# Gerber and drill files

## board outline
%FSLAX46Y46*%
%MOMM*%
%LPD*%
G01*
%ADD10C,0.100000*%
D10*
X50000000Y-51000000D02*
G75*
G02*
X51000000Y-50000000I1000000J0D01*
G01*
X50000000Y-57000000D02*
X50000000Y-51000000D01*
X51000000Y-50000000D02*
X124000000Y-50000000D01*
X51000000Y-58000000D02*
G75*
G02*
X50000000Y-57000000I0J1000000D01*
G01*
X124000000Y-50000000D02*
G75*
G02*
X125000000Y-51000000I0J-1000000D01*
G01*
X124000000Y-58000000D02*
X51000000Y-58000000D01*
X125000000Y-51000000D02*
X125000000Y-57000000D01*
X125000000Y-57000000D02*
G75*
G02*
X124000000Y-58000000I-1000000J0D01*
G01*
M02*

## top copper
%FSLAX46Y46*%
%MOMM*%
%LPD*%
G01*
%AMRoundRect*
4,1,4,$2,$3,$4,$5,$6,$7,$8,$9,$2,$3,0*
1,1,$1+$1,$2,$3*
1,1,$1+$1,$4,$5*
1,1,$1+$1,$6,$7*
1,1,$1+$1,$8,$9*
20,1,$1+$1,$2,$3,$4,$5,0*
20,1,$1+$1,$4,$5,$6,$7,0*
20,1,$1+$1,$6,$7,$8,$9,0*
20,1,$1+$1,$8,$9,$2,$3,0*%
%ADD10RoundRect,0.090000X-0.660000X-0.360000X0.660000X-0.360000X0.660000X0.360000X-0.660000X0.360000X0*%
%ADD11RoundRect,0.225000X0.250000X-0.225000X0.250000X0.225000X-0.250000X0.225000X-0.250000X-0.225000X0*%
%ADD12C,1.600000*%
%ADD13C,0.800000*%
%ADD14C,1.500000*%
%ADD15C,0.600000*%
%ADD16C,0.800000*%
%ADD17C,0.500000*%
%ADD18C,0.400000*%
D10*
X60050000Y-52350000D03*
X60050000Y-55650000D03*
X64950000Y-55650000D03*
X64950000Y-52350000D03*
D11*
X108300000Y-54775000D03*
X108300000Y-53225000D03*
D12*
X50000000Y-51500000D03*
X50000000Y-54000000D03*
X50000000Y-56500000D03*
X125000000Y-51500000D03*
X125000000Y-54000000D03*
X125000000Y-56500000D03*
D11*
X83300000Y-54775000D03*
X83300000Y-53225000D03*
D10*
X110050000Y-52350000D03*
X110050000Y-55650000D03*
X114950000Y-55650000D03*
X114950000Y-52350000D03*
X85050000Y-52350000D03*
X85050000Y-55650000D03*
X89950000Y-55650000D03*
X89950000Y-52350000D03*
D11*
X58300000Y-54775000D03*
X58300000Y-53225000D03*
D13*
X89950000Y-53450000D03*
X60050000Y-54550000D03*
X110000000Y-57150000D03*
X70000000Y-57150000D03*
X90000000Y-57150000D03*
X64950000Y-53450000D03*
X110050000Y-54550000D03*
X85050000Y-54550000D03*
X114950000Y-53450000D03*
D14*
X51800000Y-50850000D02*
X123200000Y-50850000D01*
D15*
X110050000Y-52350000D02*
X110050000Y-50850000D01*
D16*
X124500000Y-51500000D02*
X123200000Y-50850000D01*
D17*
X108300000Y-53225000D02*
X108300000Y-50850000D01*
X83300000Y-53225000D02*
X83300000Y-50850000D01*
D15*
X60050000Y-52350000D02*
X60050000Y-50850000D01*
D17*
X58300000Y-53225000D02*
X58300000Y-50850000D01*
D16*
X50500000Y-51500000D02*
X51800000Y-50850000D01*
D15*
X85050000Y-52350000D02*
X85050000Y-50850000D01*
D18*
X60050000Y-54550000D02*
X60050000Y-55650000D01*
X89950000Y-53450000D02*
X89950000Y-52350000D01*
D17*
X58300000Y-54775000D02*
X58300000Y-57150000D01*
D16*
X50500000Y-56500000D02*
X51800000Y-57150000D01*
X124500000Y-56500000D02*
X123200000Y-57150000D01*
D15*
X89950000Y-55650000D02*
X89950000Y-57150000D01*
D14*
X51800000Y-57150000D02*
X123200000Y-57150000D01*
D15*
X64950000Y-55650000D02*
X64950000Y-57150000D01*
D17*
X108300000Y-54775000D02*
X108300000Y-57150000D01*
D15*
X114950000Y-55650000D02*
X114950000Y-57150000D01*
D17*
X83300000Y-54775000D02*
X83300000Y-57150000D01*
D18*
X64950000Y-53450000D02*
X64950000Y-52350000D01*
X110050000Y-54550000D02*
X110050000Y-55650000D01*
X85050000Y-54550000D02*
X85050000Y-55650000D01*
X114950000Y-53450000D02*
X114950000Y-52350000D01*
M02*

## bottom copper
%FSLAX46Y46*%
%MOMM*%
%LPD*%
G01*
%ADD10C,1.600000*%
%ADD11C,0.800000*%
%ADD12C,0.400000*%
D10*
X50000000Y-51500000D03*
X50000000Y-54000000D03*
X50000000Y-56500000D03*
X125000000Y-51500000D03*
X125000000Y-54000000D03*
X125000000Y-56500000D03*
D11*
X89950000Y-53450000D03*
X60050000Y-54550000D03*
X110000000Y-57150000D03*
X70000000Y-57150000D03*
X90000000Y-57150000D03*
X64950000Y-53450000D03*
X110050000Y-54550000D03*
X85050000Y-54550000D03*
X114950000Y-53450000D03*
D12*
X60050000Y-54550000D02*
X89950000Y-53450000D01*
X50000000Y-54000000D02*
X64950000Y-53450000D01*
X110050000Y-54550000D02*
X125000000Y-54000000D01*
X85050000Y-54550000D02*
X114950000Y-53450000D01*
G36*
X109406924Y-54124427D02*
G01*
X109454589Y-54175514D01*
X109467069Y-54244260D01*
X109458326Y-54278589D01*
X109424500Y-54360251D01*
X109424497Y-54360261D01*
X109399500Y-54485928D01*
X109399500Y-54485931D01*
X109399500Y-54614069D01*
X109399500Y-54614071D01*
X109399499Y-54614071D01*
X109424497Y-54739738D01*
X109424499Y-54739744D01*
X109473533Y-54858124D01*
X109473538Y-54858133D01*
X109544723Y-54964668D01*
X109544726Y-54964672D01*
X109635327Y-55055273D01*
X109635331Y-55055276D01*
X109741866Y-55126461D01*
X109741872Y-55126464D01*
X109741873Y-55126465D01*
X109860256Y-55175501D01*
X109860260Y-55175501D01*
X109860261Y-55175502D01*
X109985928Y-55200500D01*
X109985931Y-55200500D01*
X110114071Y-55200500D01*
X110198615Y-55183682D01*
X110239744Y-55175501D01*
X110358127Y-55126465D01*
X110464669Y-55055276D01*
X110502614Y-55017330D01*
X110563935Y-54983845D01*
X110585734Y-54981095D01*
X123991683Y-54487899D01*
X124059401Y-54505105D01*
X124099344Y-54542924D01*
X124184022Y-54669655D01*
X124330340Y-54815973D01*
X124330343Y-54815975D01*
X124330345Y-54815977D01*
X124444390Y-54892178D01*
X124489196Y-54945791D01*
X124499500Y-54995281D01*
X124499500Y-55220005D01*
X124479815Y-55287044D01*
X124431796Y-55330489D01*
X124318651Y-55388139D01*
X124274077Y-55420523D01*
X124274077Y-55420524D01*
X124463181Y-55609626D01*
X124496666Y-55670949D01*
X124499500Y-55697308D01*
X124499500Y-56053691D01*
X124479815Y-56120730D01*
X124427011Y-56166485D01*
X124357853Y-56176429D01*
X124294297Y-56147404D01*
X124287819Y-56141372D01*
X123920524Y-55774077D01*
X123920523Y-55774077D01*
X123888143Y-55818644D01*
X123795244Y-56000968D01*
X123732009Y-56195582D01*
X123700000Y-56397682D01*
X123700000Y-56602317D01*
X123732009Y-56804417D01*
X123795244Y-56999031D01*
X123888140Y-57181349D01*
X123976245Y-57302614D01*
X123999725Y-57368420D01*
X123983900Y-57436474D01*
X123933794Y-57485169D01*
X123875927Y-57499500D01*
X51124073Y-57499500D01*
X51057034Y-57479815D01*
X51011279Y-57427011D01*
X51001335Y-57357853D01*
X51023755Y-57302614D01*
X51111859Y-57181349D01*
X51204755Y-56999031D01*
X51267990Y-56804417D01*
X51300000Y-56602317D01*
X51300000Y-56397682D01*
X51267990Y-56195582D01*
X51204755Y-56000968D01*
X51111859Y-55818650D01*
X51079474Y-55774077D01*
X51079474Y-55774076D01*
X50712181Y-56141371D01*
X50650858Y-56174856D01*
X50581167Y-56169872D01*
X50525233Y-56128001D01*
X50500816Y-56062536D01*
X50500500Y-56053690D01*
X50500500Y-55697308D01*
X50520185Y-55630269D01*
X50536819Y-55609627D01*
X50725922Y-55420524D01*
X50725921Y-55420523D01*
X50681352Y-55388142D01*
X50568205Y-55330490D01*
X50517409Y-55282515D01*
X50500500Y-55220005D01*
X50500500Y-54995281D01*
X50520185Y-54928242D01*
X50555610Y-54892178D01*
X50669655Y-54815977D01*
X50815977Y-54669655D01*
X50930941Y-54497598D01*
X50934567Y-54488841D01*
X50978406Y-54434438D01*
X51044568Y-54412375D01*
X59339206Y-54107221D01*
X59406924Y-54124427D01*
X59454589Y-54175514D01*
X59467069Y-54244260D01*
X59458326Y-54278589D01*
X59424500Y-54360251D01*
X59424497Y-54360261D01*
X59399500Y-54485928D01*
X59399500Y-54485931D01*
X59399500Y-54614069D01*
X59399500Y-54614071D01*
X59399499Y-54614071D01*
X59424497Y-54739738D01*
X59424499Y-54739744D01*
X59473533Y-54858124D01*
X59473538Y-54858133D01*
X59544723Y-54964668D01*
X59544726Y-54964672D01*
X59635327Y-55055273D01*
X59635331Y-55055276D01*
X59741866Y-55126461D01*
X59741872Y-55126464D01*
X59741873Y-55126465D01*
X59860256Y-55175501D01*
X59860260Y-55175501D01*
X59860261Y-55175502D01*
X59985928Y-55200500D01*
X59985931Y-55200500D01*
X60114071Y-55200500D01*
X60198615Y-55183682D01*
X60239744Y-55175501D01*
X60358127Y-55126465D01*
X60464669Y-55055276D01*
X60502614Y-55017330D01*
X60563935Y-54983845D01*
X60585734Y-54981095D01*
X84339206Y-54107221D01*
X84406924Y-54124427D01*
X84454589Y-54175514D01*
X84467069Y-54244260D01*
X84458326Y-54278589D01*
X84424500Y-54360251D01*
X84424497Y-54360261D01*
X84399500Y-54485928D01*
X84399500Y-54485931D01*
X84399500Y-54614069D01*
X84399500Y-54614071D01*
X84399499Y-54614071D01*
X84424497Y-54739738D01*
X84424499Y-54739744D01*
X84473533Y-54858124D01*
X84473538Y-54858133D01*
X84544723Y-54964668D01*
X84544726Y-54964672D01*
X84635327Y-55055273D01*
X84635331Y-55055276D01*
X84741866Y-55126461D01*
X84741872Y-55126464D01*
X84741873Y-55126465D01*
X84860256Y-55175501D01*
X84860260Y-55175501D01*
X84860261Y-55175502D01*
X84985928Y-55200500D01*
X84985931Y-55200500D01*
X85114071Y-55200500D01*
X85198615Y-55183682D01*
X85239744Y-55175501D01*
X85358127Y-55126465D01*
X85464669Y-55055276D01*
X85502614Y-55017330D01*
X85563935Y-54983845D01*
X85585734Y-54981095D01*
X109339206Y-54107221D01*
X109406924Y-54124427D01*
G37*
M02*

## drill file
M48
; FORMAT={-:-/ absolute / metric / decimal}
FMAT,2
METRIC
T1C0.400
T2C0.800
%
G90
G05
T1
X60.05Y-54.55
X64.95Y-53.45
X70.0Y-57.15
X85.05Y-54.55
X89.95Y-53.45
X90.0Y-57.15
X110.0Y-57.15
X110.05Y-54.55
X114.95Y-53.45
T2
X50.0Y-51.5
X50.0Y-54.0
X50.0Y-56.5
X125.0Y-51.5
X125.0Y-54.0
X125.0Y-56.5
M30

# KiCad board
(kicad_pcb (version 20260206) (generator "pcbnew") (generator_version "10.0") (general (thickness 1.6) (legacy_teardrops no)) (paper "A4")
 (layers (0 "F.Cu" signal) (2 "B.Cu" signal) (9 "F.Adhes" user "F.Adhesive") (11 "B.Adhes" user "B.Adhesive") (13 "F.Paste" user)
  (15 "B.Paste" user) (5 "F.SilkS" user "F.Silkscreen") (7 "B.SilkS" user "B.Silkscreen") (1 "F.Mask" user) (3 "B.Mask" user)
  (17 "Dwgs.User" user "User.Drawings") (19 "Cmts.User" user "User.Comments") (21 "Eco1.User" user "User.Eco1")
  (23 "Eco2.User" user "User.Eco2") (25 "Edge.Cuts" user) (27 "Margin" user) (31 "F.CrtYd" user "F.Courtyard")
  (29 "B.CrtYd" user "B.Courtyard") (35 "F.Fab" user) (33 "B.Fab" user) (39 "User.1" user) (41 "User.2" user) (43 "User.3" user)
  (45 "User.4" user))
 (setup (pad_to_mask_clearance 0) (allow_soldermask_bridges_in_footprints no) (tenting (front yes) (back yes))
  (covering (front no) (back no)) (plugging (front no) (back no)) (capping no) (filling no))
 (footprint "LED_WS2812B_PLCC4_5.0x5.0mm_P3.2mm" (layer "F.Cu") (at 62.5 54)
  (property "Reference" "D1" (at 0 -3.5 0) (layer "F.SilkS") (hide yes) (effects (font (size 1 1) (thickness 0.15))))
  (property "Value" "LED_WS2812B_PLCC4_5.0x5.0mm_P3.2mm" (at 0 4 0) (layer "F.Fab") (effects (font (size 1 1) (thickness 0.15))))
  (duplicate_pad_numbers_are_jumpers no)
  (pad "1" smd roundrect (at -2.45 -1.65) (size 1.5 0.9) (layers "F.Cu" "F.Mask" "F.Paste") (roundrect_rratio 0.1) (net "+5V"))
  (pad "2" smd roundrect (at -2.45 1.65) (size 1.5 0.9) (layers "F.Cu" "F.Mask" "F.Paste") (roundrect_rratio 0.1) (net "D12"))
  (pad "3" smd roundrect (at 2.45 1.65) (size 1.5 0.9) (layers "F.Cu" "F.Mask" "F.Paste") (roundrect_rratio 0.1) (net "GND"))
  (pad "4" smd roundrect (at 2.45 -1.65) (size 1.5 0.9) (layers "F.Cu" "F.Mask" "F.Paste") (roundrect_rratio 0.1) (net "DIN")))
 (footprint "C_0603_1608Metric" (layer "F.Cu") (at 108.3 54 90)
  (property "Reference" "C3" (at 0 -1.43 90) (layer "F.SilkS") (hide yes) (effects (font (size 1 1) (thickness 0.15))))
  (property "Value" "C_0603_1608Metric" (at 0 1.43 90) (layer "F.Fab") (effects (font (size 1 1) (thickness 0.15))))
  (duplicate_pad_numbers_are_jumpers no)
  (pad "1" smd roundrect (at -0.775 0 90) (size 0.9 0.95) (layers "F.Cu" "F.Mask" "F.Paste") (roundrect_rratio 0.25) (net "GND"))
  (pad "2" smd roundrect (at 0.775 0 90) (size 0.9 0.95) (layers "F.Cu" "F.Mask" "F.Paste") (roundrect_rratio 0.25) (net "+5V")))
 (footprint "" (layer "F.Cu") (at 50 54)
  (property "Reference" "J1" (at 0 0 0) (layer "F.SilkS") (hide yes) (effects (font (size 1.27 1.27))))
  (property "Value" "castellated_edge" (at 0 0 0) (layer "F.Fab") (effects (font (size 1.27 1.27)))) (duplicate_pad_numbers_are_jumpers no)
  (pad "1" thru_hole circle (at 0 -2.5) (size 1.6 1.6) (drill 0.8) (layers "*.Cu" "*.Mask") (remove_unused_layers no) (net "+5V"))
  (pad "2" thru_hole circle (at 0 0) (size 1.6 1.6) (drill 0.8) (layers "*.Cu" "*.Mask") (remove_unused_layers no) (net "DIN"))
  (pad "3" thru_hole circle (at 0 2.5) (size 1.6 1.6) (drill 0.8) (layers "*.Cu" "*.Mask") (remove_unused_layers no) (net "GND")))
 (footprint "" (layer "F.Cu") (at 125 54)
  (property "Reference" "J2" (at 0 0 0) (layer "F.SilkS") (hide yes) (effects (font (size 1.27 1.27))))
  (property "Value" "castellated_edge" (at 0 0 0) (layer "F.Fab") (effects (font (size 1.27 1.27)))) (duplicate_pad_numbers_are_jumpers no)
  (pad "1" thru_hole circle (at 0 -2.5) (size 1.6 1.6) (drill 0.8) (layers "*.Cu" "*.Mask") (remove_unused_layers no) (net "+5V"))
  (pad "2" thru_hole circle (at 0 0) (size 1.6 1.6) (drill 0.8) (layers "*.Cu" "*.Mask") (remove_unused_layers no) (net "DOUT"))
  (pad "3" thru_hole circle (at 0 2.5) (size 1.6 1.6) (drill 0.8) (layers "*.Cu" "*.Mask") (remove_unused_layers no) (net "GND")))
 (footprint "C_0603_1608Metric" (layer "F.Cu") (at 83.3 54 90)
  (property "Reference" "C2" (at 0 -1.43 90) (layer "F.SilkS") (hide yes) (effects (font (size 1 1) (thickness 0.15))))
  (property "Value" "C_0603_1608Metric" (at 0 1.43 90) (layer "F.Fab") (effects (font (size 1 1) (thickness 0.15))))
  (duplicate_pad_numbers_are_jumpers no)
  (pad "1" smd roundrect (at -0.775 0 90) (size 0.9 0.95) (layers "F.Cu" "F.Mask" "F.Paste") (roundrect_rratio 0.25) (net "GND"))
  (pad "2" smd roundrect (at 0.775 0 90) (size 0.9 0.95) (layers "F.Cu" "F.Mask" "F.Paste") (roundrect_rratio 0.25) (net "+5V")))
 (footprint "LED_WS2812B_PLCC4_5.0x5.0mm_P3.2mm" (layer "F.Cu") (at 112.5 54)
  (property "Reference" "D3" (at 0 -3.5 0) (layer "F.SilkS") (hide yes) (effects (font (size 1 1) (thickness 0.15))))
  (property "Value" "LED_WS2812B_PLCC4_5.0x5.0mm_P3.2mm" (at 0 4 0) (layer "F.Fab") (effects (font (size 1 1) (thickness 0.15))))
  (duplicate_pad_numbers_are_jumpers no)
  (pad "1" smd roundrect (at -2.45 -1.65) (size 1.5 0.9) (layers "F.Cu" "F.Mask" "F.Paste") (roundrect_rratio 0.1) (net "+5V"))
  (pad "2" smd roundrect (at -2.45 1.65) (size 1.5 0.9) (layers "F.Cu" "F.Mask" "F.Paste") (roundrect_rratio 0.1) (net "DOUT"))
  (pad "3" smd roundrect (at 2.45 1.65) (size 1.5 0.9) (layers "F.Cu" "F.Mask" "F.Paste") (roundrect_rratio 0.1) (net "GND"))
  (pad "4" smd roundrect (at 2.45 -1.65) (size 1.5 0.9) (layers "F.Cu" "F.Mask" "F.Paste") (roundrect_rratio 0.1) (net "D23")))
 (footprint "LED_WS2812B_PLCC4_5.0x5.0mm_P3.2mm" (layer "F.Cu") (at 87.5 54)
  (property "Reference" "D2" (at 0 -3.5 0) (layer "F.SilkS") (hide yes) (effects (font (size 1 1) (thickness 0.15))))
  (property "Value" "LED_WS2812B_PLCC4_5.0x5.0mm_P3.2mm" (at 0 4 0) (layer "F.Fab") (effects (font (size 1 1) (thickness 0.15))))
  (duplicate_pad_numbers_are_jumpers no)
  (pad "1" smd roundrect (at -2.45 -1.65) (size 1.5 0.9) (layers "F.Cu" "F.Mask" "F.Paste") (roundrect_rratio 0.1) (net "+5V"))
  (pad "2" smd roundrect (at -2.45 1.65) (size 1.5 0.9) (layers "F.Cu" "F.Mask" "F.Paste") (roundrect_rratio 0.1) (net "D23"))
  (pad "3" smd roundrect (at 2.45 1.65) (size 1.5 0.9) (layers "F.Cu" "F.Mask" "F.Paste") (roundrect_rratio 0.1) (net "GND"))
  (pad "4" smd roundrect (at 2.45 -1.65) (size 1.5 0.9) (layers "F.Cu" "F.Mask" "F.Paste") (roundrect_rratio 0.1) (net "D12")))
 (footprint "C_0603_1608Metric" (layer "F.Cu") (at 58.3 54 90)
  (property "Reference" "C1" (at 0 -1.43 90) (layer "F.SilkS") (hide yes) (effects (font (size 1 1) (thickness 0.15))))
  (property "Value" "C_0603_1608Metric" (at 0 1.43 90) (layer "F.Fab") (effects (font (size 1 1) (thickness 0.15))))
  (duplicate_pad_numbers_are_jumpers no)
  (pad "1" smd roundrect (at -0.775 0 90) (size 0.9 0.95) (layers "F.Cu" "F.Mask" "F.Paste") (roundrect_rratio 0.25) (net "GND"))
  (pad "2" smd roundrect (at 0.775 0 90) (size 0.9 0.95) (layers "F.Cu" "F.Mask" "F.Paste") (roundrect_rratio 0.25) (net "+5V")))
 (gr_arc (start 50 51) (mid 50.292893 50.292893) (end 51 50) (stroke (width 0.1) (type default)) (layer "Edge.Cuts"))
 (gr_line (start 50 57) (end 50 51) (stroke (width 0.1) (type default)) (layer "Edge.Cuts"))
 (gr_line (start 51 50) (end 124 50) (stroke (width 0.1) (type default)) (layer "Edge.Cuts"))
 (gr_arc (start 51 58) (mid 50.292893 57.707106) (end 50 57) (stroke (width 0.1) (type default)) (layer "Edge.Cuts"))
 (gr_arc (start 124 50) (mid 124.707106 50.292893) (end 125 51) (stroke (width 0.1) (type default)) (layer "Edge.Cuts"))
 (gr_line (start 124 58) (end 51 58) (stroke (width 0.1) (type default)) (layer "Edge.Cuts"))
 (gr_line (start 125 51) (end 125 57) (stroke (width 0.1) (type default)) (layer "Edge.Cuts"))
 (gr_arc (start 125 57) (mid 124.707106 57.707106) (end 124 58) (stroke (width 0.1) (type default)) (layer "Edge.Cuts"))
 (segment (start 51.8 50.85) (end 123.2 50.85) (width 1.5) (layer "F.Cu") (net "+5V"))
 (segment (start 110.05 52.35) (end 110.05 50.85) (width 0.6) (layer "F.Cu") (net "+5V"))
 (segment (start 124.5 51.5) (end 123.2 50.85) (width 0.8) (layer "F.Cu") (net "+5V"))
 (segment (start 108.3 53.225) (end 108.3 50.85) (width 0.5) (layer "F.Cu") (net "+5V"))
 (segment (start 83.3 53.225) (end 83.3 50.85) (width 0.5) (layer "F.Cu") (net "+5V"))
 (segment (start 60.05 52.35) (end 60.05 50.85) (width 0.6) (layer "F.Cu") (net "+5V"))
 (segment (start 58.3 53.225) (end 58.3 50.85) (width 0.5) (layer "F.Cu") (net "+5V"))
 (segment (start 50.5 51.5) (end 51.8 50.85) (width 0.8) (layer "F.Cu") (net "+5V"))
 (segment (start 85.05 52.35) (end 85.05 50.85) (width 0.6) (layer "F.Cu") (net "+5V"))
 (segment (start 60.05 54.55) (end 60.05 55.65) (width 0.4) (layer "F.Cu") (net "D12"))
 (segment (start 89.95 53.45) (end 89.95 52.35) (width 0.4) (layer "F.Cu") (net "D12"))
 (via (at 89.95 53.45) (size 0.8) (drill 0.4) (layers "F.Cu" "B.Cu") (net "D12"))
 (via (at 60.05 54.55) (size 0.8) (drill 0.4) (layers "F.Cu" "B.Cu") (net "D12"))
 (segment (start 60.05 54.55) (end 89.95 53.45) (width 0.4) (layer "B.Cu") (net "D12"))
 (segment (start 58.3 54.775) (end 58.3 57.15) (width 0.5) (layer "F.Cu") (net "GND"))
 (segment (start 50.5 56.5) (end 51.8 57.15) (width 0.8) (layer "F.Cu") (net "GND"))
 (segment (start 124.5 56.5) (end 123.2 57.15) (width 0.8) (layer "F.Cu") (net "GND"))
 (segment (start 89.95 55.65) (end 89.95 57.15) (width 0.6) (layer "F.Cu") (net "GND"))
 (segment (start 51.8 57.15) (end 123.2 57.15) (width 1.5) (layer "F.Cu") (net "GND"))
 (segment (start 64.95 55.65) (end 64.95 57.15) (width 0.6) (layer "F.Cu") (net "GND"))
 (segment (start 108.3 54.775) (end 108.3 57.15) (width 0.5) (layer "F.Cu") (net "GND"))
 (segment (start 114.95 55.65) (end 114.95 57.15) (width 0.6) (layer "F.Cu") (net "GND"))
 (segment (start 83.3 54.775) (end 83.3 57.15) (width 0.5) (layer "F.Cu") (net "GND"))
 (via (at 110 57.15) (size 0.8) (drill 0.4) (layers "F.Cu" "B.Cu") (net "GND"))
 (via (at 70 57.15) (size 0.8) (drill 0.4) (layers "F.Cu" "B.Cu") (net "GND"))
 (via (at 90 57.15) (size 0.8) (drill 0.4) (layers "F.Cu" "B.Cu") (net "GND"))
 (segment (start 64.95 53.45) (end 64.95 52.35) (width 0.4) (layer "F.Cu") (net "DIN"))
 (via (at 64.95 53.45) (size 0.8) (drill 0.4) (layers "F.Cu" "B.Cu") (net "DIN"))
 (segment (start 50 54) (end 64.95 53.45) (width 0.4) (layer "B.Cu") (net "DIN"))
 (segment (start 110.05 54.55) (end 110.05 55.65) (width 0.4) (layer "F.Cu") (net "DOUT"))
 (via (at 110.05 54.55) (size 0.8) (drill 0.4) (layers "F.Cu" "B.Cu") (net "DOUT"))
 (segment (start 110.05 54.55) (end 125 54) (width 0.4) (layer "B.Cu") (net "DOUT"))
 (segment (start 85.05 54.55) (end 85.05 55.65) (width 0.4) (layer "F.Cu") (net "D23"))
 (segment (start 114.95 53.45) (end 114.95 52.35) (width 0.4) (layer "F.Cu") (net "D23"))
 (via (at 85.05 54.55) (size 0.8) (drill 0.4) (layers "F.Cu" "B.Cu") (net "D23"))
 (via (at 114.95 53.45) (size 0.8) (drill 0.4) (layers "F.Cu" "B.Cu") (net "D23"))
 (segment (start 85.05 54.55) (end 114.95 53.45) (width 0.4) (layer "B.Cu") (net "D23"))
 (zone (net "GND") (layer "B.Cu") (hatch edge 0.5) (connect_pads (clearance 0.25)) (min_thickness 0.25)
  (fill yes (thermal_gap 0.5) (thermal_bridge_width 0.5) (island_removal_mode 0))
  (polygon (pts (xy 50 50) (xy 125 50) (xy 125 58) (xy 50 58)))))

